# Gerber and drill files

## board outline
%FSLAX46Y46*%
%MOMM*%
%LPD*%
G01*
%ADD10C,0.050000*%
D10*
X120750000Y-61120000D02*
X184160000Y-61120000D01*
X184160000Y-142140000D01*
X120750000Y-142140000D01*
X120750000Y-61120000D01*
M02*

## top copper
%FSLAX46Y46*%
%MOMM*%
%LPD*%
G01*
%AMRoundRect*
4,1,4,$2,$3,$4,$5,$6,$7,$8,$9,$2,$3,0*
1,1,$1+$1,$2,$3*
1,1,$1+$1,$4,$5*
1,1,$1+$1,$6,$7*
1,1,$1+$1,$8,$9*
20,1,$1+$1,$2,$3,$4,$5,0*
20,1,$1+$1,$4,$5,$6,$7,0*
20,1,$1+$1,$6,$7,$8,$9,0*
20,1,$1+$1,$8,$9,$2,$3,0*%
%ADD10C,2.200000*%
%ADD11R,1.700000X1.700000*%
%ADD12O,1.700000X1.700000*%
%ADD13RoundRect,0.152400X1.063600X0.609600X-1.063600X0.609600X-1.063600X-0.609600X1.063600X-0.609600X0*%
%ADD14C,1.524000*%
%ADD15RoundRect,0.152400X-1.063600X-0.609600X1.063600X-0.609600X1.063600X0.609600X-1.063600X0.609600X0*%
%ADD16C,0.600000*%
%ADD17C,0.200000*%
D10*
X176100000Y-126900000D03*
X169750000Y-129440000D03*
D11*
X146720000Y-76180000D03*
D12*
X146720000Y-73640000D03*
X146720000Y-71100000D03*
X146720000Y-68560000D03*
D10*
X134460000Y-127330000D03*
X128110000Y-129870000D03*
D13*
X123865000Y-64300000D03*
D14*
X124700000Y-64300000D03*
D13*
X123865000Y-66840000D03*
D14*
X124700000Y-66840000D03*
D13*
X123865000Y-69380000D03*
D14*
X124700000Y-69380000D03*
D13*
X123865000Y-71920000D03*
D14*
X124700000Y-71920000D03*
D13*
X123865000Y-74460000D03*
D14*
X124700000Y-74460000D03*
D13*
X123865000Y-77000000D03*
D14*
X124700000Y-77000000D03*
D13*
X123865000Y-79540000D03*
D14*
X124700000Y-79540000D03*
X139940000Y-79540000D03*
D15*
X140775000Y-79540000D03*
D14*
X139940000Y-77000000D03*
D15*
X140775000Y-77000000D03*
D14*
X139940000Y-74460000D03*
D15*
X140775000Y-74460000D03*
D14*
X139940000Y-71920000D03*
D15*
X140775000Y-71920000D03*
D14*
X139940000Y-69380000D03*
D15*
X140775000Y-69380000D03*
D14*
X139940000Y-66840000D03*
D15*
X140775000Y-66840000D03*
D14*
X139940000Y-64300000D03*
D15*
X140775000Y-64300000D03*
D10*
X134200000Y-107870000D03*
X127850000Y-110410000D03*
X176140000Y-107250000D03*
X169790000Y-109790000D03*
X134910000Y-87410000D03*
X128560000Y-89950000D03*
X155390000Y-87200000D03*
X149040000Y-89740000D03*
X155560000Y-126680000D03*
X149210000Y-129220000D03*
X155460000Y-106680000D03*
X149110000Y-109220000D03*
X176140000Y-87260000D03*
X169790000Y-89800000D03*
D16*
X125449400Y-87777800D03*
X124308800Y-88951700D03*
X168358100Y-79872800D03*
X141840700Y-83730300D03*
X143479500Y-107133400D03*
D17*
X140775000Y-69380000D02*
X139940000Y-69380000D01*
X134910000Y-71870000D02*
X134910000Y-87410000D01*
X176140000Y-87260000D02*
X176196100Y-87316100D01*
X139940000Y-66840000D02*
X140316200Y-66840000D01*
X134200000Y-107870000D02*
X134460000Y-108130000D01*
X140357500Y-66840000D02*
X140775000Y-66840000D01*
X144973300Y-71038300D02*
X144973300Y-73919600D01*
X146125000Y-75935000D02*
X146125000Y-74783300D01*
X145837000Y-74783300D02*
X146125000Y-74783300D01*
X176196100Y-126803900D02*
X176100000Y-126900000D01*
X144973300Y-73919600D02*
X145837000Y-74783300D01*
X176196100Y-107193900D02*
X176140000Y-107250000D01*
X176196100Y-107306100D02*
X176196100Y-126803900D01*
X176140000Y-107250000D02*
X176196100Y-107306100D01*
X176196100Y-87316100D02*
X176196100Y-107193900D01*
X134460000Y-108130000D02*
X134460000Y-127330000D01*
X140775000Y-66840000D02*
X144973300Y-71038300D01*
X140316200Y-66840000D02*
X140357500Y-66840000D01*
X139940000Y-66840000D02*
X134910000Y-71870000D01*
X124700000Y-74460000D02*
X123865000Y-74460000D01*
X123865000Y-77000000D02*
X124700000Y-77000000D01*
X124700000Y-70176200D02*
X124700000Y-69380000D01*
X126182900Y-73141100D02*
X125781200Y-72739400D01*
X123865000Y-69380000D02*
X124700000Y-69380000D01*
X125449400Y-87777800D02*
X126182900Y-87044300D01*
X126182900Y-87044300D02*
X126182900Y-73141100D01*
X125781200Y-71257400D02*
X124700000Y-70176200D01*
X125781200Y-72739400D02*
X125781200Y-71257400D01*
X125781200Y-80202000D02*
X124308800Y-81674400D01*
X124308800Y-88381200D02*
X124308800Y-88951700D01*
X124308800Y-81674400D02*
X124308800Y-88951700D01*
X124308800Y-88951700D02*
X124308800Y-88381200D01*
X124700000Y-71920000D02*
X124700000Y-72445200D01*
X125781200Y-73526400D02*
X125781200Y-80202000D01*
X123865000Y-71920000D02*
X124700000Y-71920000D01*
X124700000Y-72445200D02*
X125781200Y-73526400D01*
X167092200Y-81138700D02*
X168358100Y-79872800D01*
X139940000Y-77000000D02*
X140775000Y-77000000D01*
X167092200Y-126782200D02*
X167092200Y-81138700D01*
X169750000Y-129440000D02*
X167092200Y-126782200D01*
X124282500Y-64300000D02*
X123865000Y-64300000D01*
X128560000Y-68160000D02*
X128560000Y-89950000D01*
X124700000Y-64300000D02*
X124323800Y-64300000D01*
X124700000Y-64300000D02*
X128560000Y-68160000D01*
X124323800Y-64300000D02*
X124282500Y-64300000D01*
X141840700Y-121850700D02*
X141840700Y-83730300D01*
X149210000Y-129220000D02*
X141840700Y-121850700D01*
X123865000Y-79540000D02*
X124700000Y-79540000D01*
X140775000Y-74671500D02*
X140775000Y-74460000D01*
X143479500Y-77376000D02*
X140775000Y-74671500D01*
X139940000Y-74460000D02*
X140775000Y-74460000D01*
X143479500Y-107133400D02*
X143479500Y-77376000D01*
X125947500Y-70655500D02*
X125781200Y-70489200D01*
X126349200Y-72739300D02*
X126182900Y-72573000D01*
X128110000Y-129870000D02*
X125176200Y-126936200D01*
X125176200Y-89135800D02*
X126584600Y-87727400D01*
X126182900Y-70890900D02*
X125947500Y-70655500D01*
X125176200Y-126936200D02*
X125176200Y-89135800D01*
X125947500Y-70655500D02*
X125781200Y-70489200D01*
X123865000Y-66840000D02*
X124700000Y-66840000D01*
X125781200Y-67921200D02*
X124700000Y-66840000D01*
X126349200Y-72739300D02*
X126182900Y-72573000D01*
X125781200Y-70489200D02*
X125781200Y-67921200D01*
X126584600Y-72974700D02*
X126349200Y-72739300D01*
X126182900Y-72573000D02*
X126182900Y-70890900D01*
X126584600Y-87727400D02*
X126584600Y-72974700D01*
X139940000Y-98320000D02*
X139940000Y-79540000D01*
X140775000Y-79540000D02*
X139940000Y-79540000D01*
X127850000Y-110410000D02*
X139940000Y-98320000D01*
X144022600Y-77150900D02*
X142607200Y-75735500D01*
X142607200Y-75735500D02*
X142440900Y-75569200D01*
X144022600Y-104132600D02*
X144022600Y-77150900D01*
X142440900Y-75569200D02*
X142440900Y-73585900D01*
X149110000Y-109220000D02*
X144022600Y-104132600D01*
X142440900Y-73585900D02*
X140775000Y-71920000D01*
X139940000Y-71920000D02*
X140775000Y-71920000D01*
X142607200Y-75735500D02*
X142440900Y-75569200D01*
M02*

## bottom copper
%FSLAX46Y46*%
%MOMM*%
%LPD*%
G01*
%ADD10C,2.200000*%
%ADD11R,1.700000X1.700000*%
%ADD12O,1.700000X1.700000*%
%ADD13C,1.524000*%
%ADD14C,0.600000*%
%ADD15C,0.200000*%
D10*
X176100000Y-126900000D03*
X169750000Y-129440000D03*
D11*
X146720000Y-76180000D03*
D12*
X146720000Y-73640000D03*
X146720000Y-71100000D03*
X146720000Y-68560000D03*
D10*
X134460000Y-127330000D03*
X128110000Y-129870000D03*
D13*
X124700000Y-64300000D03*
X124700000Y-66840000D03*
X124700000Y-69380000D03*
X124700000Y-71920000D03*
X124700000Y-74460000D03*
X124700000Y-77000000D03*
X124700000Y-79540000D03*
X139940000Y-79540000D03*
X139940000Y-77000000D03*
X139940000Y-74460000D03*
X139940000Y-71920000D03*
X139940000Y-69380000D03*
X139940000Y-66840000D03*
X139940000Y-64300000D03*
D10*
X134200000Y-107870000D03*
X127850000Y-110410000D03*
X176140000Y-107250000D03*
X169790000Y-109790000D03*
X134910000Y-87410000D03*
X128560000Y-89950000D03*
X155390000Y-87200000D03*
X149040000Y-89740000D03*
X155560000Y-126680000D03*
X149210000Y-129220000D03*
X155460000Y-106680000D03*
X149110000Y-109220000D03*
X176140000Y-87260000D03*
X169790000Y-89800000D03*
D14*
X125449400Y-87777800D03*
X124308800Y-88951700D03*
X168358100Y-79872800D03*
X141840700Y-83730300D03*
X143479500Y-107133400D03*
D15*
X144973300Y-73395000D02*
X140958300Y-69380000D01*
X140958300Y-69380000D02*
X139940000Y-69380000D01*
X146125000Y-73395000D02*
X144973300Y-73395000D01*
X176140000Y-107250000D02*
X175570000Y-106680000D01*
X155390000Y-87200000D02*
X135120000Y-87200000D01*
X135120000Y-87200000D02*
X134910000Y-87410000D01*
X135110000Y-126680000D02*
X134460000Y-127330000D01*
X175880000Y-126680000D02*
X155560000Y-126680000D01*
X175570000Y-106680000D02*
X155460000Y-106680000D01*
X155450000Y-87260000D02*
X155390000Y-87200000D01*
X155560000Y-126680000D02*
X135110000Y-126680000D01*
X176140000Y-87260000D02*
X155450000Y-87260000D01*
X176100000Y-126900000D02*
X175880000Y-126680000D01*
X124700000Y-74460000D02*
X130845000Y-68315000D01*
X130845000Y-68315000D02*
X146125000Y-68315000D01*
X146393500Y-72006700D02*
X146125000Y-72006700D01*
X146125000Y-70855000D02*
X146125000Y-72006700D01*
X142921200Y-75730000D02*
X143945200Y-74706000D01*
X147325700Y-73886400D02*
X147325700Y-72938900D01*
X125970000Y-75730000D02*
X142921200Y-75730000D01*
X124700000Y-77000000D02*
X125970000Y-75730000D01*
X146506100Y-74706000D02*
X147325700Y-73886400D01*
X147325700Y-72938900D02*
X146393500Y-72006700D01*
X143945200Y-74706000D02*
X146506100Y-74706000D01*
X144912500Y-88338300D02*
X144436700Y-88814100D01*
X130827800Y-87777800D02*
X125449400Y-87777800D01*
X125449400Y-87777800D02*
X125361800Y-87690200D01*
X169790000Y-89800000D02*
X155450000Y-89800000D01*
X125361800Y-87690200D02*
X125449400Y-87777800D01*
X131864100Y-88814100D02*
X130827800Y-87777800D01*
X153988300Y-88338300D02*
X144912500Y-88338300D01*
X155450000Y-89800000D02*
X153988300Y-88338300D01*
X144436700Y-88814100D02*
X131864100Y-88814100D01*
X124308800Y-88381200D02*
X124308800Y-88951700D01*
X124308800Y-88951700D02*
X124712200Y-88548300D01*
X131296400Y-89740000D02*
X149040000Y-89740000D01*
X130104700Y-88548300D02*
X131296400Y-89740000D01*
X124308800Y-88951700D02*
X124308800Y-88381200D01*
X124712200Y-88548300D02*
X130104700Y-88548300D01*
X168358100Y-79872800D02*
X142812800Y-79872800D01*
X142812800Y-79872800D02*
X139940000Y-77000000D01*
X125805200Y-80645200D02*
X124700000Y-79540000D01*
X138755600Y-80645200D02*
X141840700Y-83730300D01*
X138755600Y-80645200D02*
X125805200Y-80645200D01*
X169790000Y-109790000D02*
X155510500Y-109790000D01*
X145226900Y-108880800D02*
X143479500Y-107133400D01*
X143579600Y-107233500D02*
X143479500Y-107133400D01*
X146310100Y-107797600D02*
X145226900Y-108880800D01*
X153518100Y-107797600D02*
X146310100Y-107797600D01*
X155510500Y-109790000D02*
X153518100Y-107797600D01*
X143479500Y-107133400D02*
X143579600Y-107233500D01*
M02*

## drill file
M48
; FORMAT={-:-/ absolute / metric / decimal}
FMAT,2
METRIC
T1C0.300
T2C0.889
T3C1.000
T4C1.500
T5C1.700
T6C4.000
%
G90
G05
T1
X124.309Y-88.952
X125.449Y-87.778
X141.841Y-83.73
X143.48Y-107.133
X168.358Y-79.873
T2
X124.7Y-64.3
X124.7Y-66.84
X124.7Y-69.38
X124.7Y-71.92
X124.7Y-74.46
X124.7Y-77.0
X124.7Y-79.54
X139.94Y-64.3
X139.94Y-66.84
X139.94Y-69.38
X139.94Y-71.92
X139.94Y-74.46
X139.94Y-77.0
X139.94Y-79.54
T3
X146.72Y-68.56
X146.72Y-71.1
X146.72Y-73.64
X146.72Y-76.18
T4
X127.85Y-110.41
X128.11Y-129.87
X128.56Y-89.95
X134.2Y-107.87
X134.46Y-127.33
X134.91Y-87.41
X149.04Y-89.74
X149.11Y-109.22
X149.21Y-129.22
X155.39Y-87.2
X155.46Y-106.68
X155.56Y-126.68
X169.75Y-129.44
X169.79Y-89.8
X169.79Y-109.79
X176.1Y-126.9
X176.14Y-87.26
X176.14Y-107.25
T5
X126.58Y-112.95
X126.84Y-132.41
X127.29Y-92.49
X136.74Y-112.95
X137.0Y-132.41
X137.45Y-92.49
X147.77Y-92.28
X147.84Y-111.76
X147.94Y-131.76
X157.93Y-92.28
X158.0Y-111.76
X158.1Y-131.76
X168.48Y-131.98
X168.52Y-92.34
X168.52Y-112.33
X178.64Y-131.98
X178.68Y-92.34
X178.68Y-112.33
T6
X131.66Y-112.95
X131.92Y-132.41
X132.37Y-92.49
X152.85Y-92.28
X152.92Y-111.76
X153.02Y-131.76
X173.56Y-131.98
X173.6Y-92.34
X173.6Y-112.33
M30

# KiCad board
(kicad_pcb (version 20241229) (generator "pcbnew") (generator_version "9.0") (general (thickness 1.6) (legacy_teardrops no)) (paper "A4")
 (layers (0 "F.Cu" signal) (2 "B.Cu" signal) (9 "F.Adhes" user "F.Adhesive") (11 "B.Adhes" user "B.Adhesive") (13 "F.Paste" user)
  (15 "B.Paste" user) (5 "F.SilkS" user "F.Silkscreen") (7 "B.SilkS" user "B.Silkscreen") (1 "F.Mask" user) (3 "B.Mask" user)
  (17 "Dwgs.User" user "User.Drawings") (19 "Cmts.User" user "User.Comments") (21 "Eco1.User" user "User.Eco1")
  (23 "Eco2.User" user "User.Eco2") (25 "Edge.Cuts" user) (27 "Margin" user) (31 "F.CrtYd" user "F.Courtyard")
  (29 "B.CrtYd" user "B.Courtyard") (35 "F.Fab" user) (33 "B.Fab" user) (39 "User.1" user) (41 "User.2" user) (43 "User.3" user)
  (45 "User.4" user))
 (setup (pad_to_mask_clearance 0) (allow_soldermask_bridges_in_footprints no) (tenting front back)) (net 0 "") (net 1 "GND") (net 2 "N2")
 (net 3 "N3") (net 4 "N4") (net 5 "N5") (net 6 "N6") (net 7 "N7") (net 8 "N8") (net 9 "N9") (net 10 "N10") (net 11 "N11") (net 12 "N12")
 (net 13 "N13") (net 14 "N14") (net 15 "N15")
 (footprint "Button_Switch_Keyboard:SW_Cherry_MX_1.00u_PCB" (layer "F.Cu") (at 176.1 126.9)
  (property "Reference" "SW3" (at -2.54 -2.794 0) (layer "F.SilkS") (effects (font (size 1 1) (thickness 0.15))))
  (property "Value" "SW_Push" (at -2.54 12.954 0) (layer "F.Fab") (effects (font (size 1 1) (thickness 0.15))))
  (pad "" np_thru_hole circle (at -7.62 5.08) (size 1.7 1.7) (drill 1.7) (layers "*.Cu" "*.Mask"))
  (pad "" np_thru_hole circle (at -2.54 5.08) (size 4 4) (drill 4) (layers "*.Cu" "*.Mask"))
  (pad "" np_thru_hole circle (at 2.54 5.08) (size 1.7 1.7) (drill 1.7) (layers "*.Cu" "*.Mask"))
  (pad "1" thru_hole circle (at 0 0) (size 2.2 2.2) (drill 1.5) (layers "*.Cu" "*.Mask") (remove_unused_layers no) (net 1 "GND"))
  (pad "2" thru_hole circle (at -6.35 2.54) (size 2.2 2.2) (drill 1.5) (layers "*.Cu" "*.Mask") (remove_unused_layers no) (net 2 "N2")))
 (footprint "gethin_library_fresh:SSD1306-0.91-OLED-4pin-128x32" (layer "F.Cu") (at 183.22 78.37 180)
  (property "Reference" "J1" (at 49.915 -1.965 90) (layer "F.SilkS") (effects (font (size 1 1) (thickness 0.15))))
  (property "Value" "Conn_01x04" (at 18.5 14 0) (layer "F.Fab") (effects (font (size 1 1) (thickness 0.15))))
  (pad "1" thru_hole rect (at 36.5 2.19 180) (size 1.7 1.7) (drill 1) (layers "*.Cu" "*.Mask") (remove_unused_layers no) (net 1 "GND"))
  (pad "2" thru_hole oval (at 36.5 4.73 180) (size 1.7 1.7) (drill 1) (layers "*.Cu" "*.Mask") (remove_unused_layers no) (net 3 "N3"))
  (pad "3" thru_hole oval (at 36.5 7.27 180) (size 1.7 1.7) (drill 1) (layers "*.Cu" "*.Mask") (remove_unused_layers no) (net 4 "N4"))
  (pad "4" thru_hole oval (at 36.5 9.81 180) (size 1.7 1.7) (drill 1) (layers "*.Cu" "*.Mask") (remove_unused_layers no) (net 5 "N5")))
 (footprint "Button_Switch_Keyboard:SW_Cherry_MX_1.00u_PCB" (layer "F.Cu") (at 134.46 127.33)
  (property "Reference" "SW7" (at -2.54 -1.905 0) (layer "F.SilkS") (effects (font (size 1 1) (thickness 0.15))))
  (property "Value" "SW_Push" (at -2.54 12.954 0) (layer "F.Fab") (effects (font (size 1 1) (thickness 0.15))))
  (pad "" np_thru_hole circle (at -7.62 5.08) (size 1.7 1.7) (drill 1.7) (layers "*.Cu" "*.Mask"))
  (pad "" np_thru_hole circle (at -2.54 5.08) (size 4 4) (drill 4) (layers "*.Cu" "*.Mask"))
  (pad "" np_thru_hole circle (at 2.54 5.08) (size 1.7 1.7) (drill 1.7) (layers "*.Cu" "*.Mask"))
  (pad "1" thru_hole circle (at 0 0) (size 2.2 2.2) (drill 1.5) (layers "*.Cu" "*.Mask") (remove_unused_layers no) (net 1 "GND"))
  (pad "2" thru_hole circle (at -6.35 2.54) (size 2.2 2.2) (drill 1.5) (layers "*.Cu" "*.Mask") (remove_unused_layers no) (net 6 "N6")))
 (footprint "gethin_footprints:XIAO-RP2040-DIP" (layer "F.Cu") (at 132.32 71.92)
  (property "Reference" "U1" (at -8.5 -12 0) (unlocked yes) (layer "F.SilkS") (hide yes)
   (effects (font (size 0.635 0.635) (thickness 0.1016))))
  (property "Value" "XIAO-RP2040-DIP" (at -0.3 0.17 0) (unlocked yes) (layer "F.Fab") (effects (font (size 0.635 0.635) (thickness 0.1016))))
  (pad "1" smd roundrect (at -8.455 -7.62 180) (size 2.432 1.524) (layers "F.Cu" "F.Mask") (roundrect_rratio 0.1) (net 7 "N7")
   (thermal_bridge_angle 45))
  (pad "1" thru_hole circle (at -7.62 -7.62 180) (size 1.524 1.524) (drill 0.889) (layers "*.Cu" "*.Mask") (remove_unused_layers no)
   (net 7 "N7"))
  (pad "2" smd roundrect (at -8.455 -5.08 180) (size 2.432 1.524) (layers "F.Cu" "F.Mask") (roundrect_rratio 0.1) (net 6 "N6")
   (thermal_bridge_angle 45))
  (pad "2" thru_hole circle (at -7.62 -5.08 180) (size 1.524 1.524) (drill 0.889) (layers "*.Cu" "*.Mask") (remove_unused_layers no)
   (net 6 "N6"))
  (pad "3" smd roundrect (at -8.455 -2.54 180) (size 2.432 1.524) (layers "F.Cu" "F.Mask") (roundrect_rratio 0.1) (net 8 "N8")
   (thermal_bridge_angle 45))
  (pad "3" thru_hole circle (at -7.62 -2.54 180) (size 1.524 1.524) (drill 0.889) (layers "*.Cu" "*.Mask") (remove_unused_layers no)
   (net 8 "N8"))
  (pad "4" smd roundrect (at -8.455 0 180) (size 2.432 1.524) (layers "F.Cu" "F.Mask") (roundrect_rratio 0.1) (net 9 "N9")
   (thermal_bridge_angle 45))
  (pad "4" thru_hole circle (at -7.62 0 180) (size 1.524 1.524) (drill 0.889) (layers "*.Cu" "*.Mask") (remove_unused_layers no)
   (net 9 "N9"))
  (pad "5" smd roundrect (at -8.455 2.54 180) (size 2.432 1.524) (layers "F.Cu" "F.Mask") (roundrect_rratio 0.1) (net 5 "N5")
   (thermal_bridge_angle 45))
  (pad "5" thru_hole circle (at -7.62 2.54 180) (size 1.524 1.524) (drill 0.889) (layers "*.Cu" "*.Mask") (remove_unused_layers no)
   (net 5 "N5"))
  (pad "6" smd roundrect (at -8.455 5.08 180) (size 2.432 1.524) (layers "F.Cu" "F.Mask") (roundrect_rratio 0.1) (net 4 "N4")
   (thermal_bridge_angle 45))
  (pad "6" thru_hole circle (at -7.62 5.08 180) (size 1.524 1.524) (drill 0.889) (layers "*.Cu" "*.Mask") (remove_unused_layers no)
   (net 4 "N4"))
  (pad "7" smd roundrect (at -8.455 7.62 180) (size 2.432 1.524) (layers "F.Cu" "F.Mask") (roundrect_rratio 0.1) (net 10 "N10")
   (thermal_bridge_angle 45))
  (pad "7" thru_hole circle (at -7.62 7.62 180) (size 1.524 1.524) (drill 0.889) (layers "*.Cu" "*.Mask") (remove_unused_layers no)
   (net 10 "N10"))
  (pad "8" thru_hole circle (at 7.62 7.62) (size 1.524 1.524) (drill 0.889) (layers "*.Cu" "*.Mask") (remove_unused_layers no)
   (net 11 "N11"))
  (pad "8" smd roundrect (at 8.455 7.62) (size 2.432 1.524) (layers "F.Cu" "F.Mask") (roundrect_rratio 0.1) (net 11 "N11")
   (thermal_bridge_angle 45))
  (pad "9" thru_hole circle (at 7.62 5.08) (size 1.524 1.524) (drill 0.889) (layers "*.Cu" "*.Mask") (remove_unused_layers no) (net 2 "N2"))
  (pad "9" smd roundrect (at 8.455 5.08) (size 2.432 1.524) (layers "F.Cu" "F.Mask") (roundrect_rratio 0.1) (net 2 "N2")
   (thermal_bridge_angle 45))
  (pad "10" thru_hole circle (at 7.62 2.54) (size 1.524 1.524) (drill 0.889) (layers "*.Cu" "*.Mask") (remove_unused_layers no)
   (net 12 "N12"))
  (pad "10" smd roundrect (at 8.455 2.54) (size 2.432 1.524) (layers "F.Cu" "F.Mask") (roundrect_rratio 0.1) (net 12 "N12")
   (thermal_bridge_angle 45))
  (pad "11" thru_hole circle (at 7.62 0) (size 1.524 1.524) (drill 0.889) (layers "*.Cu" "*.Mask") (remove_unused_layers no) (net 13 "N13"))
  (pad "11" smd roundrect (at 8.455 0) (size 2.432 1.524) (layers "F.Cu" "F.Mask") (roundrect_rratio 0.1) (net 13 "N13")
   (thermal_bridge_angle 45))
  (pad "12" thru_hole circle (at 7.62 -2.54) (size 1.524 1.524) (drill 0.889) (layers "*.Cu" "*.Mask") (remove_unused_layers no)
   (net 3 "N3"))
  (pad "12" smd roundrect (at 8.455 -2.54) (size 2.432 1.524) (layers "F.Cu" "F.Mask") (roundrect_rratio 0.1) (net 3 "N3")
   (thermal_bridge_angle 45))
  (pad "13" thru_hole circle (at 7.62 -5.08) (size 1.524 1.524) (drill 0.889) (layers "*.Cu" "*.Mask") (remove_unused_layers no)
   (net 1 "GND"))
  (pad "13" smd roundrect (at 8.455 -5.08) (size 2.432 1.524) (layers "F.Cu" "F.Mask") (roundrect_rratio 0.1) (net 1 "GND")
   (thermal_bridge_angle 45))
  (pad "14" thru_hole circle (at 7.62 -7.62) (size 1.524 1.524) (drill 0.889) (layers "*.Cu" "*.Mask") (remove_unused_layers no)
   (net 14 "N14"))
  (pad "14" smd roundrect (at 8.455 -7.62) (size 2.432 1.524) (layers "F.Cu" "F.Mask") (roundrect_rratio 0.1) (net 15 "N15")
   (thermal_bridge_angle 45)))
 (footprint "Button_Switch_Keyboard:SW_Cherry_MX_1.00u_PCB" (layer "F.Cu") (at 134.2 107.87)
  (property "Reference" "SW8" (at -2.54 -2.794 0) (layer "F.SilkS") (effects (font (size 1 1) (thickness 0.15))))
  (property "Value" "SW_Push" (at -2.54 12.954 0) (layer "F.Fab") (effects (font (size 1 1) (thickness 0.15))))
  (pad "" np_thru_hole circle (at -7.62 5.08) (size 1.7 1.7) (drill 1.7) (layers "*.Cu" "*.Mask"))
  (pad "" np_thru_hole circle (at -2.54 5.08) (size 4 4) (drill 4) (layers "*.Cu" "*.Mask"))
  (pad "" np_thru_hole circle (at 2.54 5.08) (size 1.7 1.7) (drill 1.7) (layers "*.Cu" "*.Mask"))
  (pad "1" thru_hole circle (at 0 0) (size 2.2 2.2) (drill 1.5) (layers "*.Cu" "*.Mask") (remove_unused_layers no) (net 1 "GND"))
  (pad "2" thru_hole circle (at -6.35 2.54) (size 2.2 2.2) (drill 1.5) (layers "*.Cu" "*.Mask") (remove_unused_layers no) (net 11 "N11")))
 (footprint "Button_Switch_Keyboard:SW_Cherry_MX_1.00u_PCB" (layer "F.Cu") (at 176.14 107.25)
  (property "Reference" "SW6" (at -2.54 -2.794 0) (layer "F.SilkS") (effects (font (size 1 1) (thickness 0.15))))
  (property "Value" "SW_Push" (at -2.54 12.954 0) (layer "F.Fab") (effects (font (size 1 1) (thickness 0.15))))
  (pad "" np_thru_hole circle (at -7.62 5.08) (size 1.7 1.7) (drill 1.7) (layers "*.Cu" "*.Mask"))
  (pad "" np_thru_hole circle (at -2.54 5.08) (size 4 4) (drill 4) (layers "*.Cu" "*.Mask"))
  (pad "" np_thru_hole circle (at 2.54 5.08) (size 1.7 1.7) (drill 1.7) (layers "*.Cu" "*.Mask"))
  (pad "1" thru_hole circle (at 0 0) (size 2.2 2.2) (drill 1.5) (layers "*.Cu" "*.Mask") (remove_unused_layers no) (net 1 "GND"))
  (pad "2" thru_hole circle (at -6.35 2.54) (size 2.2 2.2) (drill 1.5) (layers "*.Cu" "*.Mask") (remove_unused_layers no) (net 12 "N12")))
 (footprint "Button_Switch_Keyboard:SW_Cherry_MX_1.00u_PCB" (layer "F.Cu") (at 134.91 87.41)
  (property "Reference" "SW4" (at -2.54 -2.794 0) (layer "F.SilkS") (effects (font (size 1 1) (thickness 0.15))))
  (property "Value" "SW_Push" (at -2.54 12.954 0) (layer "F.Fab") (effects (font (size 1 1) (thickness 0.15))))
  (pad "" np_thru_hole circle (at -7.62 5.08) (size 1.7 1.7) (drill 1.7) (layers "*.Cu" "*.Mask"))
  (pad "" np_thru_hole circle (at -2.54 5.08) (size 4 4) (drill 4) (layers "*.Cu" "*.Mask"))
  (pad "" np_thru_hole circle (at 2.54 5.08) (size 1.7 1.7) (drill 1.7) (layers "*.Cu" "*.Mask"))
  (pad "1" thru_hole circle (at 0 0) (size 2.2 2.2) (drill 1.5) (layers "*.Cu" "*.Mask") (remove_unused_layers no) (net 1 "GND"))
  (pad "2" thru_hole circle (at -6.35 2.54) (size 2.2 2.2) (drill 1.5) (layers "*.Cu" "*.Mask") (remove_unused_layers no) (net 7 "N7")))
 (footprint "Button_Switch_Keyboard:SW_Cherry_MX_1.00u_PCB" (layer "F.Cu") (at 155.39 87.2)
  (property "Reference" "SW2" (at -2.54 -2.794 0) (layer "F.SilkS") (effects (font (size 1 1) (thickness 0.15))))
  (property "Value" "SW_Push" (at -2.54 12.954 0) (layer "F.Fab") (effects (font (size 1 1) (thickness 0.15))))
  (pad "" np_thru_hole circle (at -7.62 5.08) (size 1.7 1.7) (drill 1.7) (layers "*.Cu" "*.Mask"))
  (pad "" np_thru_hole circle (at -2.54 5.08) (size 4 4) (drill 4) (layers "*.Cu" "*.Mask"))
  (pad "" np_thru_hole circle (at 2.54 5.08) (size 1.7 1.7) (drill 1.7) (layers "*.Cu" "*.Mask"))
  (pad "1" thru_hole circle (at 0 0) (size 2.2 2.2) (drill 1.5) (layers "*.Cu" "*.Mask") (remove_unused_layers no) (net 1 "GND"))
  (pad "2" thru_hole circle (at -6.35 2.54) (size 2.2 2.2) (drill 1.5) (layers "*.Cu" "*.Mask") (remove_unused_layers no) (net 9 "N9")))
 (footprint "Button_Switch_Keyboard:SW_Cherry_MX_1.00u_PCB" (layer "F.Cu") (at 155.56 126.68)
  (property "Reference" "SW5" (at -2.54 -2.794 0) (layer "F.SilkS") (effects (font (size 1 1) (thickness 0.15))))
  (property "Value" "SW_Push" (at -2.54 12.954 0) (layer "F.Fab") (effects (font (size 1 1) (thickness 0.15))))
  (pad "" np_thru_hole circle (at -7.62 5.08) (size 1.7 1.7) (drill 1.7) (layers "*.Cu" "*.Mask"))
  (pad "" np_thru_hole circle (at -2.54 5.08) (size 4 4) (drill 4) (layers "*.Cu" "*.Mask"))
  (pad "" np_thru_hole circle (at 2.54 5.08) (size 1.7 1.7) (drill 1.7) (layers "*.Cu" "*.Mask"))
  (pad "1" thru_hole circle (at 0 0) (size 2.2 2.2) (drill 1.5) (layers "*.Cu" "*.Mask") (remove_unused_layers no) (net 1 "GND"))
  (pad "2" thru_hole circle (at -6.35 2.54) (size 2.2 2.2) (drill 1.5) (layers "*.Cu" "*.Mask") (remove_unused_layers no) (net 10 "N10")))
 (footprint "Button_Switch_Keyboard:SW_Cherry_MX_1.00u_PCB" (layer "F.Cu") (at 155.46 106.68)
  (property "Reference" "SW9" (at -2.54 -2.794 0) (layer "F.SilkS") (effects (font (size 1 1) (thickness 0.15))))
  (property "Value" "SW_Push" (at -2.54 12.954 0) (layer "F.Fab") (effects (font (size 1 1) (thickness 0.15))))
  (pad "" np_thru_hole circle (at -7.62 5.08) (size 1.7 1.7) (drill 1.7) (layers "*.Cu" "*.Mask"))
  (pad "" np_thru_hole circle (at -2.54 5.08) (size 4 4) (drill 4) (layers "*.Cu" "*.Mask"))
  (pad "" np_thru_hole circle (at 2.54 5.08) (size 1.7 1.7) (drill 1.7) (layers "*.Cu" "*.Mask"))
  (pad "1" thru_hole circle (at 0 0) (size 2.2 2.2) (drill 1.5) (layers "*.Cu" "*.Mask") (remove_unused_layers no) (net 1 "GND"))
  (pad "2" thru_hole circle (at -6.35 2.54) (size 2.2 2.2) (drill 1.5) (layers "*.Cu" "*.Mask") (remove_unused_layers no) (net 13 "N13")))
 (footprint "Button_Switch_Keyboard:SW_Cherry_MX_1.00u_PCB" (layer "F.Cu") (at 176.14 87.26)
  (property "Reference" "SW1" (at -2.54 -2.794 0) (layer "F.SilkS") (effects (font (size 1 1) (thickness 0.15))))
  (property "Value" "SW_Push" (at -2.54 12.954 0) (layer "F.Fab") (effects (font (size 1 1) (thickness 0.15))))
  (pad "" np_thru_hole circle (at -7.62 5.08) (size 1.7 1.7) (drill 1.7) (layers "*.Cu" "*.Mask"))
  (pad "" np_thru_hole circle (at -2.54 5.08) (size 4 4) (drill 4) (layers "*.Cu" "*.Mask"))
  (pad "" np_thru_hole circle (at 2.54 5.08) (size 1.7 1.7) (drill 1.7) (layers "*.Cu" "*.Mask"))
  (pad "1" thru_hole circle (at 0 0) (size 2.2 2.2) (drill 1.5) (layers "*.Cu" "*.Mask") (remove_unused_layers no) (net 1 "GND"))
  (pad "2" thru_hole circle (at -6.35 2.54) (size 2.2 2.2) (drill 1.5) (layers "*.Cu" "*.Mask") (remove_unused_layers no) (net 8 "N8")))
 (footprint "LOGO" (layer "B.Cu") (at 134.62 69.55 180)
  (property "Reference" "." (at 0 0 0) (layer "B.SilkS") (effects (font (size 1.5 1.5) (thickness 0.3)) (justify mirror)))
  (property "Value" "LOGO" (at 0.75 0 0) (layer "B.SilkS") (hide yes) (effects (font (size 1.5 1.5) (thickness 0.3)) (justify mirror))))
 (gr_rect (start 120.75 61.12) (end 184.16 142.14) (stroke (width 0.05) (type default)) (fill no) (layer "Edge.Cuts"))
 (segment (start 140.775 69.38) (end 139.94 69.38) (width 0.2) (layer "F.Cu") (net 3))
 (segment (start 144.9733 73.395) (end 140.9583 69.38) (width 0.2) (layer "B.Cu") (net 3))
 (segment (start 140.9583 69.38) (end 139.94 69.38) (width 0.2) (layer "B.Cu") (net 3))
 (segment (start 146.125 73.395) (end 144.9733 73.395) (width 0.2) (layer "B.Cu") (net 3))
 (segment (start 134.91 71.87) (end 134.91 87.41) (width 0.2) (layer "F.Cu") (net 1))
 (segment (start 176.14 87.26) (end 176.1961 87.3161) (width 0.2) (layer "F.Cu") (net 1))
 (segment (start 139.94 66.84) (end 140.3162 66.84) (width 0.2) (layer "F.Cu") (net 1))
 (segment (start 134.2 107.87) (end 134.46 108.13) (width 0.2) (layer "F.Cu") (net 1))
 (segment (start 140.3575 66.84) (end 140.775 66.84) (width 0.2) (layer "F.Cu") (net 1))
 (segment (start 144.9733 71.0383) (end 144.9733 73.9196) (width 0.2) (layer "F.Cu") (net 1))
 (segment (start 146.125 75.935) (end 146.125 74.7833) (width 0.2) (layer "F.Cu") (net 1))
 (segment (start 145.837 74.7833) (end 146.125 74.7833) (width 0.2) (layer "F.Cu") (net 1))
 (segment (start 176.1961 126.8039) (end 176.1 126.9) (width 0.2) (layer "F.Cu") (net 1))
 (segment (start 144.9733 73.9196) (end 145.837 74.7833) (width 0.2) (layer "F.Cu") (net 1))
 (segment (start 176.1961 107.1939) (end 176.14 107.25) (width 0.2) (layer "F.Cu") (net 1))
 (segment (start 176.1961 107.3061) (end 176.1961 126.8039) (width 0.2) (layer "F.Cu") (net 1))
 (segment (start 176.14 107.25) (end 176.1961 107.3061) (width 0.2) (layer "F.Cu") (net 1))
 (segment (start 176.1961 87.3161) (end 176.1961 107.1939) (width 0.2) (layer "F.Cu") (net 1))
 (segment (start 134.46 108.13) (end 134.46 127.33) (width 0.2) (layer "F.Cu") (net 1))
 (segment (start 140.775 66.84) (end 144.9733 71.0383) (width 0.2) (layer "F.Cu") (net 1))
 (segment (start 140.3162 66.84) (end 140.3575 66.84) (width 0.2) (layer "F.Cu") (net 1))
 (segment (start 139.94 66.84) (end 134.91 71.87) (width 0.2) (layer "F.Cu") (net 1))
 (segment (start 176.14 107.25) (end 175.57 106.68) (width 0.2) (layer "B.Cu") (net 1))
 (segment (start 155.39 87.2) (end 135.12 87.2) (width 0.2) (layer "B.Cu") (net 1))
 (segment (start 135.12 87.2) (end 134.91 87.41) (width 0.2) (layer "B.Cu") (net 1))
 (segment (start 135.11 126.68) (end 134.46 127.33) (width 0.2) (layer "B.Cu") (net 1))
 (segment (start 175.88 126.68) (end 155.56 126.68) (width 0.2) (layer "B.Cu") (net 1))
 (segment (start 175.57 106.68) (end 155.46 106.68) (width 0.2) (layer "B.Cu") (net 1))
 (segment (start 155.45 87.26) (end 155.39 87.2) (width 0.2) (layer "B.Cu") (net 1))
 (segment (start 155.56 126.68) (end 135.11 126.68) (width 0.2) (layer "B.Cu") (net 1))
 (segment (start 176.14 87.26) (end 155.45 87.26) (width 0.2) (layer "B.Cu") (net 1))
 (segment (start 176.1 126.9) (end 175.88 126.68) (width 0.2) (layer "B.Cu") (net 1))
 (segment (start 124.7 74.46) (end 123.865 74.46) (width 0.2) (layer "F.Cu") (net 5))
 (segment (start 124.7 74.46) (end 130.845 68.315) (width 0.2) (layer "B.Cu") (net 5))
 (segment (start 130.845 68.315) (end 146.125 68.315) (width 0.2) (layer "B.Cu") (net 5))
 (segment (start 123.865 77) (end 124.7 77) (width 0.2) (layer "F.Cu") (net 4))
 (segment (start 146.3935 72.0067) (end 146.125 72.0067) (width 0.2) (layer "B.Cu") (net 4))
 (segment (start 146.125 70.855) (end 146.125 72.0067) (width 0.2) (layer "B.Cu") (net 4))
 (segment (start 142.9212 75.73) (end 143.9452 74.706) (width 0.2) (layer "B.Cu") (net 4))
 (segment (start 147.3257 73.8864) (end 147.3257 72.9389) (width 0.2) (layer "B.Cu") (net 4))
 (segment (start 125.97 75.73) (end 142.9212 75.73) (width 0.2) (layer "B.Cu") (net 4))
 (segment (start 124.7 77) (end 125.97 75.73) (width 0.2) (layer "B.Cu") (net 4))
 (segment (start 146.5061 74.706) (end 147.3257 73.8864) (width 0.2) (layer "B.Cu") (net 4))
 (segment (start 147.3257 72.9389) (end 146.3935 72.0067) (width 0.2) (layer "B.Cu") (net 4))
 (segment (start 143.9452 74.706) (end 146.5061 74.706) (width 0.2) (layer "B.Cu") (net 4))
 (segment (start 124.7 70.1762) (end 124.7 69.38) (width 0.2) (layer "F.Cu") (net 8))
 (segment (start 126.1829 73.1411) (end 125.7812 72.7394) (width 0.2) (layer "F.Cu") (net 8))
 (segment (start 123.865 69.38) (end 124.7 69.38) (width 0.2) (layer "F.Cu") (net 8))
 (segment (start 125.4494 87.7778) (end 126.1829 87.0443) (width 0.2) (layer "F.Cu") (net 8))
 (segment (start 126.1829 87.0443) (end 126.1829 73.1411) (width 0.2) (layer "F.Cu") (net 8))
 (segment (start 125.7812 71.2574) (end 124.7 70.1762) (width 0.2) (layer "F.Cu") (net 8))
 (segment (start 125.7812 72.7394) (end 125.7812 71.2574) (width 0.2) (layer "F.Cu") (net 8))
 (via (at 125.4494 87.7778) (size 0.6) (drill 0.3) (layers "F.Cu" "B.Cu") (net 8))
 (segment (start 144.9125 88.3383) (end 144.4367 88.8141) (width 0.2) (layer "B.Cu") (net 8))
 (segment (start 130.8278 87.7778) (end 125.4494 87.7778) (width 0.2) (layer "B.Cu") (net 8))
 (segment (start 125.4494 87.7778) (end 125.3618 87.6902) (width 0.2) (layer "B.Cu") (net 8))
 (segment (start 169.79 89.8) (end 155.45 89.8) (width 0.2) (layer "B.Cu") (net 8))
 (segment (start 125.3618 87.6902) (end 125.4494 87.7778) (width 0.2) (layer "B.Cu") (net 8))
 (segment (start 131.8641 88.8141) (end 130.8278 87.7778) (width 0.2) (layer "B.Cu") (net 8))
 (segment (start 153.9883 88.3383) (end 144.9125 88.3383) (width 0.2) (layer "B.Cu") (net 8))
 (segment (start 155.45 89.8) (end 153.9883 88.3383) (width 0.2) (layer "B.Cu") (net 8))
 (segment (start 144.4367 88.8141) (end 131.8641 88.8141) (width 0.2) (layer "B.Cu") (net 8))
 (segment (start 125.7812 80.202) (end 124.3088 81.6744) (width 0.2) (layer "F.Cu") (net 9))
 (segment (start 124.3088 88.3812) (end 124.3088 88.9517) (width 0.2) (layer "F.Cu") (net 9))
 (segment (start 124.3088 81.6744) (end 124.3088 88.9517) (width 0.2) (layer "F.Cu") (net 9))
 (segment (start 124.3088 88.9517) (end 124.3088 88.3812) (width 0.2) (layer "F.Cu") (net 9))
 (segment (start 124.7 71.92) (end 124.7 72.4452) (width 0.2) (layer "F.Cu") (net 9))
 (segment (start 125.7812 73.5264) (end 125.7812 80.202) (width 0.2) (layer "F.Cu") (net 9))
 (segment (start 123.865 71.92) (end 124.7 71.92) (width 0.2) (layer "F.Cu") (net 9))
 (segment (start 124.7 72.4452) (end 125.7812 73.5264) (width 0.2) (layer "F.Cu") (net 9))
 (via (at 124.3088 88.9517) (size 0.6) (drill 0.3) (layers "F.Cu" "B.Cu") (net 9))
 (segment (start 124.3088 88.3812) (end 124.3088 88.9517) (width 0.2) (layer "B.Cu") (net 9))
 (segment (start 124.3088 88.9517) (end 124.7122 88.5483) (width 0.2) (layer "B.Cu") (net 9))
 (segment (start 131.2964 89.74) (end 149.04 89.74) (width 0.2) (layer "B.Cu") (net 9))
 (segment (start 130.1047 88.5483) (end 131.2964 89.74) (width 0.2) (layer "B.Cu") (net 9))
 (segment (start 124.3088 88.9517) (end 124.3088 88.3812) (width 0.2) (layer "B.Cu") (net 9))
 (segment (start 124.7122 88.5483) (end 130.1047 88.5483) (width 0.2) (layer "B.Cu") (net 9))
 (segment (start 167.0922 81.1387) (end 168.3581 79.8728) (width 0.2) (layer "F.Cu") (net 2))
 (segment (start 139.94 77) (end 140.775 77) (width 0.2) (layer "F.Cu") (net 2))
 (segment (start 167.0922 126.7822) (end 167.0922 81.1387) (width 0.2) (layer "F.Cu") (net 2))
 (segment (start 169.75 129.44) (end 167.0922 126.7822) (width 0.2) (layer "F.Cu") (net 2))
 (via (at 168.3581 79.8728) (size 0.6) (drill 0.3) (layers "F.Cu" "B.Cu") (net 2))
 (segment (start 168.3581 79.8728) (end 142.8128 79.8728) (width 0.2) (layer "B.Cu") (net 2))
 (segment (start 142.8128 79.8728) (end 139.94 77) (width 0.2) (layer "B.Cu") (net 2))
 (segment (start 124.2825 64.3) (end 123.865 64.3) (width 0.2) (layer "F.Cu") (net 7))
 (segment (start 128.56 68.16) (end 128.56 89.95) (width 0.2) (layer "F.Cu") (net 7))
 (segment (start 124.7 64.3) (end 124.3238 64.3) (width 0.2) (layer "F.Cu") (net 7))
 (segment (start 124.7 64.3) (end 128.56 68.16) (width 0.2) (layer "F.Cu") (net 7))
 (segment (start 124.3238 64.3) (end 124.2825 64.3) (width 0.2) (layer "F.Cu") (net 7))
 (segment (start 141.8407 121.8507) (end 141.8407 83.7303) (width 0.2) (layer "F.Cu") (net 10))
 (segment (start 149.21 129.22) (end 141.8407 121.8507) (width 0.2) (layer "F.Cu") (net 10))
 (segment (start 123.865 79.54) (end 124.7 79.54) (width 0.2) (layer "F.Cu") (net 10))
 (via (at 141.8407 83.7303) (size 0.6) (drill 0.3) (layers "F.Cu" "B.Cu") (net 10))
 (segment (start 125.8052 80.6452) (end 124.7 79.54) (width 0.2) (layer "B.Cu") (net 10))
 (segment (start 138.7556 80.6452) (end 141.8407 83.7303) (width 0.2) (layer "B.Cu") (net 10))
 (segment (start 138.7556 80.6452) (end 125.8052 80.6452) (width 0.2) (layer "B.Cu") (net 10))
 (segment (start 140.775 74.6715) (end 140.775 74.46) (width 0.2) (layer "F.Cu") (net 12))
 (segment (start 143.4795 77.376) (end 140.775 74.6715) (width 0.2) (layer "F.Cu") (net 12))
 (segment (start 139.94 74.46) (end 140.775 74.46) (width 0.2) (layer "F.Cu") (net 12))
 (segment (start 143.4795 107.1334) (end 143.4795 77.376) (width 0.2) (layer "F.Cu") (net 12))
 (via (at 143.4795 107.1334) (size 0.6) (drill 0.3) (layers "F.Cu" "B.Cu") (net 12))
 (segment (start 169.79 109.79) (end 155.5105 109.79) (width 0.2) (layer "B.Cu") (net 12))
 (segment (start 145.2269 108.8808) (end 143.4795 107.1334) (width 0.2) (layer "B.Cu") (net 12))
 (segment (start 143.5796 107.2335) (end 143.4795 107.1334) (width 0.2) (layer "B.Cu") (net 12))
 (segment (start 146.3101 107.7976) (end 145.2269 108.8808) (width 0.2) (layer "B.Cu") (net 12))
 (segment (start 153.5181 107.7976) (end 146.3101 107.7976) (width 0.2) (layer "B.Cu") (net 12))
 (segment (start 155.5105 109.79) (end 153.5181 107.7976) (width 0.2) (layer "B.Cu") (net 12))
 (segment (start 143.4795 107.1334) (end 143.5796 107.2335) (width 0.2) (layer "B.Cu") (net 12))
 (segment (start 125.9475 70.6555) (end 125.7812 70.4892) (width 0.2) (layer "F.Cu") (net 6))
 (segment (start 126.3492 72.7393) (end 126.1829 72.573) (width 0.2) (layer "F.Cu") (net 6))
 (segment (start 128.11 129.87) (end 125.1762 126.9362) (width 0.2) (layer "F.Cu") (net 6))
 (segment (start 125.1762 89.1358) (end 126.5846 87.7274) (width 0.2) (layer "F.Cu") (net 6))
 (segment (start 126.1829 70.8909) (end 125.9475 70.6555) (width 0.2) (layer "F.Cu") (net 6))
 (segment (start 125.1762 126.9362) (end 125.1762 89.1358) (width 0.2) (layer "F.Cu") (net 6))
 (segment (start 125.9475 70.6555) (end 125.7812 70.4892) (width 0.2) (layer "F.Cu") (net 6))
 (segment (start 123.865 66.84) (end 124.7 66.84) (width 0.2) (layer "F.Cu") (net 6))
 (segment (start 125.7812 67.9212) (end 124.7 66.84) (width 0.2) (layer "F.Cu") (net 6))
 (segment (start 126.3492 72.7393) (end 126.1829 72.573) (width 0.2) (layer "F.Cu") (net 6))
 (segment (start 125.7812 70.4892) (end 125.7812 67.9212) (width 0.2) (layer "F.Cu") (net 6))
 (segment (start 126.5846 72.9747) (end 126.3492 72.7393) (width 0.2) (layer "F.Cu") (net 6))
 (segment (start 126.1829 72.573) (end 126.1829 70.8909) (width 0.2) (layer "F.Cu") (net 6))
 (segment (start 126.5846 87.7274) (end 126.5846 72.9747) (width 0.2) (layer "F.Cu") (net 6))
 (segment (start 139.94 98.32) (end 139.94 79.54) (width 0.2) (layer "F.Cu") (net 11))
 (segment (start 140.775 79.54) (end 139.94 79.54) (width 0.2) (layer "F.Cu") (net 11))
 (segment (start 127.85 110.41) (end 139.94 98.32) (width 0.2) (layer "F.Cu") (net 11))
 (segment (start 144.0226 77.1509) (end 142.6072 75.7355) (width 0.2) (layer "F.Cu") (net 13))
 (segment (start 142.6072 75.7355) (end 142.4409 75.5692) (width 0.2) (layer "F.Cu") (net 13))
 (segment (start 144.0226 104.1326) (end 144.0226 77.1509) (width 0.2) (layer "F.Cu") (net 13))
 (segment (start 142.4409 75.5692) (end 142.4409 73.5859) (width 0.2) (layer "F.Cu") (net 13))
 (segment (start 149.11 109.22) (end 144.0226 104.1326) (width 0.2) (layer "F.Cu") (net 13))
 (segment (start 142.4409 73.5859) (end 140.775 71.92) (width 0.2) (layer "F.Cu") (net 13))
 (segment (start 139.94 71.92) (end 140.775 71.92) (width 0.2) (layer "F.Cu") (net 13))
 (segment (start 142.6072 75.7355) (end 142.4409 75.5692) (width 0.2) (layer "F.Cu") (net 13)))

